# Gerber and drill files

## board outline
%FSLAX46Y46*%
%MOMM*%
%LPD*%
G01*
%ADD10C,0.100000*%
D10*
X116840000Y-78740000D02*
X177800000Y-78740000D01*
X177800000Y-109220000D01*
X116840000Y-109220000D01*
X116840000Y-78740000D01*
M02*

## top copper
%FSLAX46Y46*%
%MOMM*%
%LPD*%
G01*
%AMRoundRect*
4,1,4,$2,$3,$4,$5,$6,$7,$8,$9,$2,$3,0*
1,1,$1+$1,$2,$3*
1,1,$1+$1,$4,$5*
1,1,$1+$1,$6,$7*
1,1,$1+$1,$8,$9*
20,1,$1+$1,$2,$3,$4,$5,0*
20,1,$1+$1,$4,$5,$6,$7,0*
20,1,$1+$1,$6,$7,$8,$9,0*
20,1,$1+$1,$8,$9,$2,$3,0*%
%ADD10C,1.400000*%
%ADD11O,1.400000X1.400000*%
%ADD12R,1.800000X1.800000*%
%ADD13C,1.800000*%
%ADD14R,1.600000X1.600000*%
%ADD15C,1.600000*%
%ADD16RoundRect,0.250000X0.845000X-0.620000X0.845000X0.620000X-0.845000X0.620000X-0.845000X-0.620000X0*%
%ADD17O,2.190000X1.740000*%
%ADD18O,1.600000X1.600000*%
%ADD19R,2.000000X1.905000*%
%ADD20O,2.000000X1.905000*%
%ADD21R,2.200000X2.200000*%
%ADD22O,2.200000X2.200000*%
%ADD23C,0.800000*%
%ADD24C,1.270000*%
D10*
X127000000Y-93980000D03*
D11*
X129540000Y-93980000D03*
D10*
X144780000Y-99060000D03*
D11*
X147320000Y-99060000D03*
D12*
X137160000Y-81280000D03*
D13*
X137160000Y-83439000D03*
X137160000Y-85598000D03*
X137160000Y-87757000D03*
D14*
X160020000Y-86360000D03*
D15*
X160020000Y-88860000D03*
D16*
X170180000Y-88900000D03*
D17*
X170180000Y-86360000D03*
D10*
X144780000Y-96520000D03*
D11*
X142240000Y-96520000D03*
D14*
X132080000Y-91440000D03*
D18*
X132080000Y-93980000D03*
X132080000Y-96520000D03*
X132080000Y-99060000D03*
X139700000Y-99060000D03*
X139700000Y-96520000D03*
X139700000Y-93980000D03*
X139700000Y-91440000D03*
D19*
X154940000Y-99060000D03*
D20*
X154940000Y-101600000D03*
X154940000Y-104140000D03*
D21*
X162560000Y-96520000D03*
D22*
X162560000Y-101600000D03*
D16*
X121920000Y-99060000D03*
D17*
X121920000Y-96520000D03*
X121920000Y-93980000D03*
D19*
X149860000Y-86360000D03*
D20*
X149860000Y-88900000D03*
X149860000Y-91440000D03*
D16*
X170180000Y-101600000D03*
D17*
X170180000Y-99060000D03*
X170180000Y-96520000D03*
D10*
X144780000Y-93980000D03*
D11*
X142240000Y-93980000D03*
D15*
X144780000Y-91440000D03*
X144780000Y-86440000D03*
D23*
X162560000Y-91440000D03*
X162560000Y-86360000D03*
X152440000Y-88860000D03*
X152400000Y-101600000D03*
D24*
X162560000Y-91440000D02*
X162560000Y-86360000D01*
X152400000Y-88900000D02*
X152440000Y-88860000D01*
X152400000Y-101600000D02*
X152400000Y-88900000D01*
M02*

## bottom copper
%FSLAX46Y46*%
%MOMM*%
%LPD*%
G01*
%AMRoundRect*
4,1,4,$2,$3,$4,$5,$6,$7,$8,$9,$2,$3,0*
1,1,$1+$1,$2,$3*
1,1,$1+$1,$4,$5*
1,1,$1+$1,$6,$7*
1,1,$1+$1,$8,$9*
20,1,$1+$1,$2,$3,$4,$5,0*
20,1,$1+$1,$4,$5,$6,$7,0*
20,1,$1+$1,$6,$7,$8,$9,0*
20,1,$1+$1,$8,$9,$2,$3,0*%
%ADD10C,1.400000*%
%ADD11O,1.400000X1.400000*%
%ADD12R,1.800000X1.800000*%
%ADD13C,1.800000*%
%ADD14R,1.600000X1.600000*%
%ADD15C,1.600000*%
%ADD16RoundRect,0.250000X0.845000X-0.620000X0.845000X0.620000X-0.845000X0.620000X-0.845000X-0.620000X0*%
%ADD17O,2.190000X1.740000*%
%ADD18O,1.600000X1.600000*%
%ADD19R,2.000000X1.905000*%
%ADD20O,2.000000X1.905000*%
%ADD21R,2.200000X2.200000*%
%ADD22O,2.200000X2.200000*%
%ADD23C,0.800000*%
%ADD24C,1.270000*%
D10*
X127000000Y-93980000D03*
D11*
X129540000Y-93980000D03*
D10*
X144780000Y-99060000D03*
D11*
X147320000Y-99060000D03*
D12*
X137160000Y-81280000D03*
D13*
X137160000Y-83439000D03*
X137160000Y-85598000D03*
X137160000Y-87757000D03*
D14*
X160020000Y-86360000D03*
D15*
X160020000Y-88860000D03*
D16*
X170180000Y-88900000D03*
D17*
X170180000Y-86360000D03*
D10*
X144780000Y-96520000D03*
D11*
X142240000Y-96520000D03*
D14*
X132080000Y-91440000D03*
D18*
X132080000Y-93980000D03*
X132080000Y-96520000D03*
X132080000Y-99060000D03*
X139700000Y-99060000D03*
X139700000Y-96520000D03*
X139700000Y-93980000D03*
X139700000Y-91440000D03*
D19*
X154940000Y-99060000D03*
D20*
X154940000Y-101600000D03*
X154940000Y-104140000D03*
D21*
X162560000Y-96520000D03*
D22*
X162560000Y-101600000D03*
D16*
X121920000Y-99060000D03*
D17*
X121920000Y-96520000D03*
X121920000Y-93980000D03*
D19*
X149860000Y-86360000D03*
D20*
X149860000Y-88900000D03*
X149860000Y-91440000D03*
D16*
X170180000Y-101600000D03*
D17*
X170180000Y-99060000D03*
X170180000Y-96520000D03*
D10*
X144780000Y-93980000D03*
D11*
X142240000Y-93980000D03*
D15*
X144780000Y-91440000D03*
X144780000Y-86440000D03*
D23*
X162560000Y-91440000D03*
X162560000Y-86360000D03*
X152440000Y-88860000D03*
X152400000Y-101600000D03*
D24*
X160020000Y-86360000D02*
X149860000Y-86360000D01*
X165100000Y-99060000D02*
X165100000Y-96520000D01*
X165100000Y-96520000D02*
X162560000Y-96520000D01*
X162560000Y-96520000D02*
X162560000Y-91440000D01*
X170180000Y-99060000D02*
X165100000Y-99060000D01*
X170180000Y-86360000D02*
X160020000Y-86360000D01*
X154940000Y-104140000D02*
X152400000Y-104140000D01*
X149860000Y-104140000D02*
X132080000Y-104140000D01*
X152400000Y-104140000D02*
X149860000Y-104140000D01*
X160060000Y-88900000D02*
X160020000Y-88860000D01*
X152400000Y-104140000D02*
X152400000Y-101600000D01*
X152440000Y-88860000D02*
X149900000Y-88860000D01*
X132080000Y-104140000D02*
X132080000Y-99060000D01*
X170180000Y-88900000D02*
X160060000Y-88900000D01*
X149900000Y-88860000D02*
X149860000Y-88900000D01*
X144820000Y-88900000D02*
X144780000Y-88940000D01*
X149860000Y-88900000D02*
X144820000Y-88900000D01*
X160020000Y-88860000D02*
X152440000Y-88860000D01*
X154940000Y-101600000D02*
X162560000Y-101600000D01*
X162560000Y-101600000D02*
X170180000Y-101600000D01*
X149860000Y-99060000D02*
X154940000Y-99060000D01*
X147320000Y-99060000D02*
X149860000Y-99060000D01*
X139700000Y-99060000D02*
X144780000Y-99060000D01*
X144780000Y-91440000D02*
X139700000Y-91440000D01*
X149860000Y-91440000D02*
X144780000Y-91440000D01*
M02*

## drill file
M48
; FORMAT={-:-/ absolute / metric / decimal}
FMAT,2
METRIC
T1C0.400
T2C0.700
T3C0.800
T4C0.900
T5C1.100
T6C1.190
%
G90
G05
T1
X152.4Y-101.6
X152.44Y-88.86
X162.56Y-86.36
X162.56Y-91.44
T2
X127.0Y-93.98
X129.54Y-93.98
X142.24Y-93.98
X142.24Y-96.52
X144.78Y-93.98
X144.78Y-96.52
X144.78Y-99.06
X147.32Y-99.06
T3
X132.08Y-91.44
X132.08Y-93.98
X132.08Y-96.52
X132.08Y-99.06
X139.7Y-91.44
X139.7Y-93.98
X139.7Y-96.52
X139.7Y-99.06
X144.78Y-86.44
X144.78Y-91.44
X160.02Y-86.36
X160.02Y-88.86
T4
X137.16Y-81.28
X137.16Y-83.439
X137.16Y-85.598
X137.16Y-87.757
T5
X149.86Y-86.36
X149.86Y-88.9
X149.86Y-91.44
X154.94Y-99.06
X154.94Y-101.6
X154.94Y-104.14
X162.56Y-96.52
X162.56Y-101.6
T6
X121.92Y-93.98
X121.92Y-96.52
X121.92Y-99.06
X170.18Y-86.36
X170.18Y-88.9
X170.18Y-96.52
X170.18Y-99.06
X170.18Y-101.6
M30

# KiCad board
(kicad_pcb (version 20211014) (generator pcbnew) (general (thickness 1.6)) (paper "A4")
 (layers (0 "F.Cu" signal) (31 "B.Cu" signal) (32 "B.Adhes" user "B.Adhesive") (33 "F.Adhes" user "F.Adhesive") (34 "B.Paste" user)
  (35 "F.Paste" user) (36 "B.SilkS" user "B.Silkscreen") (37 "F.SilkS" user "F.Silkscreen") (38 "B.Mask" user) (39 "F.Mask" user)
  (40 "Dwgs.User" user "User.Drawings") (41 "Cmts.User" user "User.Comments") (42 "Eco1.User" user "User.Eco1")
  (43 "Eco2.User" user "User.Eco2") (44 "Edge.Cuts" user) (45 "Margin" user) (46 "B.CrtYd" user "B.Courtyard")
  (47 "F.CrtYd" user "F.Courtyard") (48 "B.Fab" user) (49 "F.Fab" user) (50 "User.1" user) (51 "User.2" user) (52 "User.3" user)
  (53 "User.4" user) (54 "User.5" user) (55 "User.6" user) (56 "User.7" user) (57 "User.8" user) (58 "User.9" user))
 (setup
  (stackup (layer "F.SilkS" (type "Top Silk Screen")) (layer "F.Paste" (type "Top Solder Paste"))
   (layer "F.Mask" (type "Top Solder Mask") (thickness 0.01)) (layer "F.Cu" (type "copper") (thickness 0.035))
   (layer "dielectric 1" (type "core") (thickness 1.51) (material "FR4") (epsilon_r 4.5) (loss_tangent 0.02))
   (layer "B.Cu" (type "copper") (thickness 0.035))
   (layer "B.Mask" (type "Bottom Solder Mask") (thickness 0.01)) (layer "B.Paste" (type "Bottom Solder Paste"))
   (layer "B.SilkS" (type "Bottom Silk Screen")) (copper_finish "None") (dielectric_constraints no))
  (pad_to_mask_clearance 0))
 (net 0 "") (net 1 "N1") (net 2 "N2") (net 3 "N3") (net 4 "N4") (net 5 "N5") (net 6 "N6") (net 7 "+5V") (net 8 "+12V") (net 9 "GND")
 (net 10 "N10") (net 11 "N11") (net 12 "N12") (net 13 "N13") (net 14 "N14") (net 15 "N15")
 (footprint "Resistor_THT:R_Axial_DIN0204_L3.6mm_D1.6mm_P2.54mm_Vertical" (layer "F.Cu") (at 127 93.98)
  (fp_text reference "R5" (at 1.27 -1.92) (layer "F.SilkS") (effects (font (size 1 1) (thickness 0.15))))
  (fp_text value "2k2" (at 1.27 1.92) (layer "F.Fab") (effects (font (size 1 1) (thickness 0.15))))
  (pad "1" thru_hole circle (at 0 0) (size 1.4 1.4) (drill 0.7) (layers *.Cu *.Mask) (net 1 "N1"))
  (pad "2" thru_hole oval (at 2.54 0) (size 1.4 1.4) (drill 0.7) (layers *.Cu *.Mask) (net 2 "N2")))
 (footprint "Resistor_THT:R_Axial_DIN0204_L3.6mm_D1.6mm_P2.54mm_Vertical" (layer "F.Cu") (at 144.78 99.06)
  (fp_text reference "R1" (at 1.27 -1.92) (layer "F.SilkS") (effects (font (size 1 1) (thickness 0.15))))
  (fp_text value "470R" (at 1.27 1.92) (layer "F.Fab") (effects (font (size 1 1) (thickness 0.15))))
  (pad "1" thru_hole circle (at 0 0) (size 1.4 1.4) (drill 0.7) (layers *.Cu *.Mask) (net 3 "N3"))
  (pad "2" thru_hole oval (at 2.54 0) (size 1.4 1.4) (drill 0.7) (layers *.Cu *.Mask) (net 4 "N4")))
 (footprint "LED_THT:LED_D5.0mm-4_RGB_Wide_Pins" (layer "F.Cu") (at 137.16 81.28 -90)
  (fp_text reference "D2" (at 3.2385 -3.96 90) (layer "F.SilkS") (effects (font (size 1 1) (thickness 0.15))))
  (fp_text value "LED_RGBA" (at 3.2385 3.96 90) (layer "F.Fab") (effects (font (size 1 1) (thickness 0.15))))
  (pad "1" thru_hole rect (at 0 0 270) (size 1.8 1.8) (drill 0.9) (layers *.Cu *.Mask) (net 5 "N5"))
  (pad "2" thru_hole circle (at 2.159 0 270) (size 1.8 1.8) (drill 0.9) (layers *.Cu *.Mask) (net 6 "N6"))
  (pad "3" thru_hole circle (at 4.318 0 270) (size 1.8 1.8) (drill 0.9) (layers *.Cu *.Mask) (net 1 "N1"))
  (pad "4" thru_hole circle (at 6.477 0 270) (size 1.8 1.8) (drill 0.9) (layers *.Cu *.Mask) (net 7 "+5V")))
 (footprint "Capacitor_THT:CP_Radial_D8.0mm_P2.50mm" (layer "F.Cu") (at 160.02 86.36 -90)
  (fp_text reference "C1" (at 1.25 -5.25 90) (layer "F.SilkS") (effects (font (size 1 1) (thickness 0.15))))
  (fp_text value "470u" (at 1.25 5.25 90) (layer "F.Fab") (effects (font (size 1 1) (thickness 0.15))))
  (pad "1" thru_hole rect (at 0 0 270) (size 1.6 1.6) (drill 0.8) (layers *.Cu *.Mask) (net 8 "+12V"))
  (pad "2" thru_hole circle (at 2.5 0 270) (size 1.6 1.6) (drill 0.8) (layers *.Cu *.Mask) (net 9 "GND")))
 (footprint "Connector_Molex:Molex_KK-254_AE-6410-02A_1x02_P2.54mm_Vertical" (layer "F.Cu") (at 170.18 88.9 90)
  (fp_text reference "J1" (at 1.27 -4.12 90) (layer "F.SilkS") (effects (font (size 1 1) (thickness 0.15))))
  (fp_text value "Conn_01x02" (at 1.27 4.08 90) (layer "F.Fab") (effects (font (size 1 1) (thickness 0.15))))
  (pad "1" thru_hole roundrect (at 0 0 90) (size 1.74 2.19) (drill 1.19) (layers *.Cu *.Mask) (roundrect_rratio 0.143678) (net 9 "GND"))
  (pad "2" thru_hole oval (at 2.54 0 90) (size 1.74 2.19) (drill 1.19) (layers *.Cu *.Mask) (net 8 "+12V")))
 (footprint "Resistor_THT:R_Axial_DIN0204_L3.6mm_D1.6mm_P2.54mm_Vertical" (layer "F.Cu") (at 144.78 96.52 180)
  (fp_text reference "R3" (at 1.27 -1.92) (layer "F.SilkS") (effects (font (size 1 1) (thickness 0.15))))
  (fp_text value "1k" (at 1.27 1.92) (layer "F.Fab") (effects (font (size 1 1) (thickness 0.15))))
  (pad "1" thru_hole circle (at 0 0 180) (size 1.4 1.4) (drill 0.7) (layers *.Cu *.Mask) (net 5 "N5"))
  (pad "2" thru_hole oval (at 2.54 0 180) (size 1.4 1.4) (drill 0.7) (layers *.Cu *.Mask) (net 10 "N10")))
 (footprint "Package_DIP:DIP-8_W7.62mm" (layer "F.Cu") (at 132.08 91.44)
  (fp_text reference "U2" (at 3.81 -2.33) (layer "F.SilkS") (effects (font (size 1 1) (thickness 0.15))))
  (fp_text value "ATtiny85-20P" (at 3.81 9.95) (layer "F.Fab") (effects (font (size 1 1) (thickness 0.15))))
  (pad "1" thru_hole rect (at 0 0) (size 1.6 1.6) (drill 0.8) (layers *.Cu *.Mask) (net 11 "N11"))
  (pad "2" thru_hole oval (at 0 2.54) (size 1.6 1.6) (drill 0.8) (layers *.Cu *.Mask) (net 2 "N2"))
  (pad "3" thru_hole oval (at 0 5.08) (size 1.6 1.6) (drill 0.8) (layers *.Cu *.Mask) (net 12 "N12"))
  (pad "4" thru_hole oval (at 0 7.62) (size 1.6 1.6) (drill 0.8) (layers *.Cu *.Mask) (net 9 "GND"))
  (pad "5" thru_hole oval (at 7.62 7.62) (size 1.6 1.6) (drill 0.8) (layers *.Cu *.Mask) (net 3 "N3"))
  (pad "6" thru_hole oval (at 7.62 5.08) (size 1.6 1.6) (drill 0.8) (layers *.Cu *.Mask) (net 10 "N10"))
  (pad "7" thru_hole oval (at 7.62 2.54) (size 1.6 1.6) (drill 0.8) (layers *.Cu *.Mask) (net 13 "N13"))
  (pad "8" thru_hole oval (at 7.62 0) (size 1.6 1.6) (drill 0.8) (layers *.Cu *.Mask) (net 7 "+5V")))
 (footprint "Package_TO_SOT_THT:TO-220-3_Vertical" (layer "F.Cu") (at 154.94 99.06 -90)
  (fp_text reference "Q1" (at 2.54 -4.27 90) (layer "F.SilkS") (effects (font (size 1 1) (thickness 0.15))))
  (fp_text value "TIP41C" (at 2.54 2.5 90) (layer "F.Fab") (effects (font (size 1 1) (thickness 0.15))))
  (pad "1" thru_hole rect (at 0 0 270) (size 1.905 2) (drill 1.1) (layers *.Cu *.Mask) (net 4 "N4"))
  (pad "2" thru_hole oval (at 2.54 0 270) (size 1.905 2) (drill 1.1) (layers *.Cu *.Mask) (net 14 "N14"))
  (pad "3" thru_hole oval (at 5.08 0 270) (size 1.905 2) (drill 1.1) (layers *.Cu *.Mask) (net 9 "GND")))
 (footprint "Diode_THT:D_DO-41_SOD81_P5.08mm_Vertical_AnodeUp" (layer "F.Cu") (at 162.56 96.52 -90)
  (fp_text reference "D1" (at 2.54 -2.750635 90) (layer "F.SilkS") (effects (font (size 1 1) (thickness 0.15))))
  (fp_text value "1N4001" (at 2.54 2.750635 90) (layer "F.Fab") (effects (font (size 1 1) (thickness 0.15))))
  (pad "1" thru_hole rect (at 0 0 270) (size 2.2 2.2) (drill 1.1) (layers *.Cu *.Mask) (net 8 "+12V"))
  (pad "2" thru_hole oval (at 5.08 0 270) (size 2.2 2.2) (drill 1.1) (layers *.Cu *.Mask) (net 14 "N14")))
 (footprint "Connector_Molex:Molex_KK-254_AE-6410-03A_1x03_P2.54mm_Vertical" (layer "F.Cu") (at 121.92 99.06 90)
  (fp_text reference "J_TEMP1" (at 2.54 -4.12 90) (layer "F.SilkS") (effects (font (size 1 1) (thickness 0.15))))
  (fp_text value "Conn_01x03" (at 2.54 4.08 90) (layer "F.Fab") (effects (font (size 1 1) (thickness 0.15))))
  (pad "1" thru_hole roundrect (at 0 0 90) (size 1.74 2.19) (drill 1.19) (layers *.Cu *.Mask) (roundrect_rratio 0.143678) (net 9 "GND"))
  (pad "2" thru_hole oval (at 2.54 0 90) (size 1.74 2.19) (drill 1.19) (layers *.Cu *.Mask) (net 12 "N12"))
  (pad "3" thru_hole oval (at 5.08 0 90) (size 1.74 2.19) (drill 1.19) (layers *.Cu *.Mask) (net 7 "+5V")))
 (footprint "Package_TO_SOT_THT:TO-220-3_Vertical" (layer "F.Cu") (at 149.86 86.36 -90)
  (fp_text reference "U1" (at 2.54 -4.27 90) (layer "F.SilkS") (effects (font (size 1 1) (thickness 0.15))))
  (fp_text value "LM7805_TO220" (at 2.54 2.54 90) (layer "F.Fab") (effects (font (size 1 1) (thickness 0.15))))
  (pad "1" thru_hole rect (at 0 0 270) (size 1.905 2) (drill 1.1) (layers *.Cu *.Mask) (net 8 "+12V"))
  (pad "2" thru_hole oval (at 2.54 0 270) (size 1.905 2) (drill 1.1) (layers *.Cu *.Mask) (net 9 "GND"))
  (pad "3" thru_hole oval (at 5.08 0 270) (size 1.905 2) (drill 1.1) (layers *.Cu *.Mask) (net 7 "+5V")))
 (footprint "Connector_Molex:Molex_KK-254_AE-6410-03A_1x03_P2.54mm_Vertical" (layer "F.Cu") (at 170.18 101.6 90)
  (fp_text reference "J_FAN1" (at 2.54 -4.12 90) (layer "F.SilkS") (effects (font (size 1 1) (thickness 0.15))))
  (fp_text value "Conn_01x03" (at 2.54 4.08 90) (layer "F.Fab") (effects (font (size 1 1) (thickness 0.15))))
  (pad "1" thru_hole roundrect (at 0 0 90) (size 1.74 2.19) (drill 1.19) (layers *.Cu *.Mask) (roundrect_rratio 0.143678) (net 14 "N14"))
  (pad "2" thru_hole oval (at 2.54 0 90) (size 1.74 2.19) (drill 1.19) (layers *.Cu *.Mask) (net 8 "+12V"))
  (pad "3" thru_hole oval (at 5.08 0 90) (size 1.74 2.19) (drill 1.19) (layers *.Cu *.Mask) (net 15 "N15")))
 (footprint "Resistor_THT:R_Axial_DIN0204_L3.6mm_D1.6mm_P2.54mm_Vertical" (layer "F.Cu") (at 144.78 93.98 180)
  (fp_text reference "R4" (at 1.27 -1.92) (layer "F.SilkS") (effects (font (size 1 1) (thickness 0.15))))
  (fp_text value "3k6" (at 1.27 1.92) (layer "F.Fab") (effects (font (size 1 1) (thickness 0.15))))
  (pad "1" thru_hole circle (at 0 0 180) (size 1.4 1.4) (drill 0.7) (layers *.Cu *.Mask) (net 6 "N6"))
  (pad "2" thru_hole oval (at 2.54 0 180) (size 1.4 1.4) (drill 0.7) (layers *.Cu *.Mask) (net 13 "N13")))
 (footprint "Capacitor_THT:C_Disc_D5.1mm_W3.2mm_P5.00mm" (layer "F.Cu") (at 144.78 91.44 90)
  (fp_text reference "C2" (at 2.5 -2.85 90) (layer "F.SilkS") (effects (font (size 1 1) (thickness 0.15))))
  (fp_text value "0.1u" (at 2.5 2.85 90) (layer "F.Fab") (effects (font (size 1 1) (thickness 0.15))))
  (pad "1" thru_hole circle (at 0 0 90) (size 1.6 1.6) (drill 0.8) (layers *.Cu *.Mask) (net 7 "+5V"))
  (pad "2" thru_hole circle (at 5 0 90) (size 1.6 1.6) (drill 0.8) (layers *.Cu *.Mask) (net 9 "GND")))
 (gr_rect (start 116.84 78.74) (end 177.8 109.22) (layer "Edge.Cuts") (width 0.1) (fill none))
 (segment (start 162.56 91.44) (end 162.56 86.36) (width 1.27) (layer "F.Cu") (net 8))
 (via (at 162.56 91.44) (size 0.8) (drill 0.4) (layers "F.Cu" "B.Cu") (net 8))
 (via (at 162.56 86.36) (size 0.8) (drill 0.4) (layers "F.Cu" "B.Cu") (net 8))
 (segment (start 160.02 86.36) (end 149.86 86.36) (width 1.27) (layer "B.Cu") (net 8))
 (segment (start 165.1 99.06) (end 165.1 96.52) (width 1.27) (layer "B.Cu") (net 8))
 (segment (start 165.1 96.52) (end 162.56 96.52) (width 1.27) (layer "B.Cu") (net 8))
 (segment (start 162.56 96.52) (end 162.56 91.44) (width 1.27) (layer "B.Cu") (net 8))
 (segment (start 170.18 99.06) (end 165.1 99.06) (width 1.27) (layer "B.Cu") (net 8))
 (segment (start 170.18 86.36) (end 160.02 86.36) (width 1.27) (layer "B.Cu") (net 8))
 (segment (start 152.4 88.9) (end 152.44 88.86) (width 1.27) (layer "F.Cu") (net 9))
 (segment (start 152.4 101.6) (end 152.4 88.9) (width 1.27) (layer "F.Cu") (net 9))
 (via (at 152.44 88.86) (size 0.8) (drill 0.4) (layers "F.Cu" "B.Cu") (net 9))
 (via (at 152.4 101.6) (size 0.8) (drill 0.4) (layers "F.Cu" "B.Cu") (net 9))
 (segment (start 154.94 104.14) (end 152.4 104.14) (width 1.27) (layer "B.Cu") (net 9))
 (segment (start 149.86 104.14) (end 132.08 104.14) (width 1.27) (layer "B.Cu") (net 9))
 (segment (start 152.4 104.14) (end 149.86 104.14) (width 1.27) (layer "B.Cu") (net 9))
 (segment (start 160.06 88.9) (end 160.02 88.86) (width 1.27) (layer "B.Cu") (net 9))
 (segment (start 152.4 104.14) (end 152.4 101.6) (width 1.27) (layer "B.Cu") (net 9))
 (segment (start 152.44 88.86) (end 149.9 88.86) (width 1.27) (layer "B.Cu") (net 9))
 (segment (start 132.08 104.14) (end 132.08 99.06) (width 1.27) (layer "B.Cu") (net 9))
 (segment (start 170.18 88.9) (end 160.06 88.9) (width 1.27) (layer "B.Cu") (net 9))
 (segment (start 149.9 88.86) (end 149.86 88.9) (width 1.27) (layer "B.Cu") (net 9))
 (segment (start 144.82 88.9) (end 144.78 88.94) (width 1.27) (layer "B.Cu") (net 9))
 (segment (start 149.86 88.9) (end 144.82 88.9) (width 1.27) (layer "B.Cu") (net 9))
 (segment (start 160.02 88.86) (end 152.44 88.86) (width 1.27) (layer "B.Cu") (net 9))
 (segment (start 154.94 101.6) (end 162.56 101.6) (width 1.27) (layer "B.Cu") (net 14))
 (segment (start 162.56 101.6) (end 170.18 101.6) (width 1.27) (layer "B.Cu") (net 14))
 (segment (start 149.86 99.06) (end 154.94 99.06) (width 1.27) (layer "B.Cu") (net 4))
 (segment (start 147.32 99.06) (end 149.86 99.06) (width 1.27) (layer "B.Cu") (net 4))
 (segment (start 139.7 99.06) (end 144.78 99.06) (width 1.27) (layer "B.Cu") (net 3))
 (segment (start 144.78 91.44) (end 139.7 91.44) (width 1.27) (layer "B.Cu") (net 7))
 (segment (start 149.86 91.44) (end 144.78 91.44) (width 1.27) (layer "B.Cu") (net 7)))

